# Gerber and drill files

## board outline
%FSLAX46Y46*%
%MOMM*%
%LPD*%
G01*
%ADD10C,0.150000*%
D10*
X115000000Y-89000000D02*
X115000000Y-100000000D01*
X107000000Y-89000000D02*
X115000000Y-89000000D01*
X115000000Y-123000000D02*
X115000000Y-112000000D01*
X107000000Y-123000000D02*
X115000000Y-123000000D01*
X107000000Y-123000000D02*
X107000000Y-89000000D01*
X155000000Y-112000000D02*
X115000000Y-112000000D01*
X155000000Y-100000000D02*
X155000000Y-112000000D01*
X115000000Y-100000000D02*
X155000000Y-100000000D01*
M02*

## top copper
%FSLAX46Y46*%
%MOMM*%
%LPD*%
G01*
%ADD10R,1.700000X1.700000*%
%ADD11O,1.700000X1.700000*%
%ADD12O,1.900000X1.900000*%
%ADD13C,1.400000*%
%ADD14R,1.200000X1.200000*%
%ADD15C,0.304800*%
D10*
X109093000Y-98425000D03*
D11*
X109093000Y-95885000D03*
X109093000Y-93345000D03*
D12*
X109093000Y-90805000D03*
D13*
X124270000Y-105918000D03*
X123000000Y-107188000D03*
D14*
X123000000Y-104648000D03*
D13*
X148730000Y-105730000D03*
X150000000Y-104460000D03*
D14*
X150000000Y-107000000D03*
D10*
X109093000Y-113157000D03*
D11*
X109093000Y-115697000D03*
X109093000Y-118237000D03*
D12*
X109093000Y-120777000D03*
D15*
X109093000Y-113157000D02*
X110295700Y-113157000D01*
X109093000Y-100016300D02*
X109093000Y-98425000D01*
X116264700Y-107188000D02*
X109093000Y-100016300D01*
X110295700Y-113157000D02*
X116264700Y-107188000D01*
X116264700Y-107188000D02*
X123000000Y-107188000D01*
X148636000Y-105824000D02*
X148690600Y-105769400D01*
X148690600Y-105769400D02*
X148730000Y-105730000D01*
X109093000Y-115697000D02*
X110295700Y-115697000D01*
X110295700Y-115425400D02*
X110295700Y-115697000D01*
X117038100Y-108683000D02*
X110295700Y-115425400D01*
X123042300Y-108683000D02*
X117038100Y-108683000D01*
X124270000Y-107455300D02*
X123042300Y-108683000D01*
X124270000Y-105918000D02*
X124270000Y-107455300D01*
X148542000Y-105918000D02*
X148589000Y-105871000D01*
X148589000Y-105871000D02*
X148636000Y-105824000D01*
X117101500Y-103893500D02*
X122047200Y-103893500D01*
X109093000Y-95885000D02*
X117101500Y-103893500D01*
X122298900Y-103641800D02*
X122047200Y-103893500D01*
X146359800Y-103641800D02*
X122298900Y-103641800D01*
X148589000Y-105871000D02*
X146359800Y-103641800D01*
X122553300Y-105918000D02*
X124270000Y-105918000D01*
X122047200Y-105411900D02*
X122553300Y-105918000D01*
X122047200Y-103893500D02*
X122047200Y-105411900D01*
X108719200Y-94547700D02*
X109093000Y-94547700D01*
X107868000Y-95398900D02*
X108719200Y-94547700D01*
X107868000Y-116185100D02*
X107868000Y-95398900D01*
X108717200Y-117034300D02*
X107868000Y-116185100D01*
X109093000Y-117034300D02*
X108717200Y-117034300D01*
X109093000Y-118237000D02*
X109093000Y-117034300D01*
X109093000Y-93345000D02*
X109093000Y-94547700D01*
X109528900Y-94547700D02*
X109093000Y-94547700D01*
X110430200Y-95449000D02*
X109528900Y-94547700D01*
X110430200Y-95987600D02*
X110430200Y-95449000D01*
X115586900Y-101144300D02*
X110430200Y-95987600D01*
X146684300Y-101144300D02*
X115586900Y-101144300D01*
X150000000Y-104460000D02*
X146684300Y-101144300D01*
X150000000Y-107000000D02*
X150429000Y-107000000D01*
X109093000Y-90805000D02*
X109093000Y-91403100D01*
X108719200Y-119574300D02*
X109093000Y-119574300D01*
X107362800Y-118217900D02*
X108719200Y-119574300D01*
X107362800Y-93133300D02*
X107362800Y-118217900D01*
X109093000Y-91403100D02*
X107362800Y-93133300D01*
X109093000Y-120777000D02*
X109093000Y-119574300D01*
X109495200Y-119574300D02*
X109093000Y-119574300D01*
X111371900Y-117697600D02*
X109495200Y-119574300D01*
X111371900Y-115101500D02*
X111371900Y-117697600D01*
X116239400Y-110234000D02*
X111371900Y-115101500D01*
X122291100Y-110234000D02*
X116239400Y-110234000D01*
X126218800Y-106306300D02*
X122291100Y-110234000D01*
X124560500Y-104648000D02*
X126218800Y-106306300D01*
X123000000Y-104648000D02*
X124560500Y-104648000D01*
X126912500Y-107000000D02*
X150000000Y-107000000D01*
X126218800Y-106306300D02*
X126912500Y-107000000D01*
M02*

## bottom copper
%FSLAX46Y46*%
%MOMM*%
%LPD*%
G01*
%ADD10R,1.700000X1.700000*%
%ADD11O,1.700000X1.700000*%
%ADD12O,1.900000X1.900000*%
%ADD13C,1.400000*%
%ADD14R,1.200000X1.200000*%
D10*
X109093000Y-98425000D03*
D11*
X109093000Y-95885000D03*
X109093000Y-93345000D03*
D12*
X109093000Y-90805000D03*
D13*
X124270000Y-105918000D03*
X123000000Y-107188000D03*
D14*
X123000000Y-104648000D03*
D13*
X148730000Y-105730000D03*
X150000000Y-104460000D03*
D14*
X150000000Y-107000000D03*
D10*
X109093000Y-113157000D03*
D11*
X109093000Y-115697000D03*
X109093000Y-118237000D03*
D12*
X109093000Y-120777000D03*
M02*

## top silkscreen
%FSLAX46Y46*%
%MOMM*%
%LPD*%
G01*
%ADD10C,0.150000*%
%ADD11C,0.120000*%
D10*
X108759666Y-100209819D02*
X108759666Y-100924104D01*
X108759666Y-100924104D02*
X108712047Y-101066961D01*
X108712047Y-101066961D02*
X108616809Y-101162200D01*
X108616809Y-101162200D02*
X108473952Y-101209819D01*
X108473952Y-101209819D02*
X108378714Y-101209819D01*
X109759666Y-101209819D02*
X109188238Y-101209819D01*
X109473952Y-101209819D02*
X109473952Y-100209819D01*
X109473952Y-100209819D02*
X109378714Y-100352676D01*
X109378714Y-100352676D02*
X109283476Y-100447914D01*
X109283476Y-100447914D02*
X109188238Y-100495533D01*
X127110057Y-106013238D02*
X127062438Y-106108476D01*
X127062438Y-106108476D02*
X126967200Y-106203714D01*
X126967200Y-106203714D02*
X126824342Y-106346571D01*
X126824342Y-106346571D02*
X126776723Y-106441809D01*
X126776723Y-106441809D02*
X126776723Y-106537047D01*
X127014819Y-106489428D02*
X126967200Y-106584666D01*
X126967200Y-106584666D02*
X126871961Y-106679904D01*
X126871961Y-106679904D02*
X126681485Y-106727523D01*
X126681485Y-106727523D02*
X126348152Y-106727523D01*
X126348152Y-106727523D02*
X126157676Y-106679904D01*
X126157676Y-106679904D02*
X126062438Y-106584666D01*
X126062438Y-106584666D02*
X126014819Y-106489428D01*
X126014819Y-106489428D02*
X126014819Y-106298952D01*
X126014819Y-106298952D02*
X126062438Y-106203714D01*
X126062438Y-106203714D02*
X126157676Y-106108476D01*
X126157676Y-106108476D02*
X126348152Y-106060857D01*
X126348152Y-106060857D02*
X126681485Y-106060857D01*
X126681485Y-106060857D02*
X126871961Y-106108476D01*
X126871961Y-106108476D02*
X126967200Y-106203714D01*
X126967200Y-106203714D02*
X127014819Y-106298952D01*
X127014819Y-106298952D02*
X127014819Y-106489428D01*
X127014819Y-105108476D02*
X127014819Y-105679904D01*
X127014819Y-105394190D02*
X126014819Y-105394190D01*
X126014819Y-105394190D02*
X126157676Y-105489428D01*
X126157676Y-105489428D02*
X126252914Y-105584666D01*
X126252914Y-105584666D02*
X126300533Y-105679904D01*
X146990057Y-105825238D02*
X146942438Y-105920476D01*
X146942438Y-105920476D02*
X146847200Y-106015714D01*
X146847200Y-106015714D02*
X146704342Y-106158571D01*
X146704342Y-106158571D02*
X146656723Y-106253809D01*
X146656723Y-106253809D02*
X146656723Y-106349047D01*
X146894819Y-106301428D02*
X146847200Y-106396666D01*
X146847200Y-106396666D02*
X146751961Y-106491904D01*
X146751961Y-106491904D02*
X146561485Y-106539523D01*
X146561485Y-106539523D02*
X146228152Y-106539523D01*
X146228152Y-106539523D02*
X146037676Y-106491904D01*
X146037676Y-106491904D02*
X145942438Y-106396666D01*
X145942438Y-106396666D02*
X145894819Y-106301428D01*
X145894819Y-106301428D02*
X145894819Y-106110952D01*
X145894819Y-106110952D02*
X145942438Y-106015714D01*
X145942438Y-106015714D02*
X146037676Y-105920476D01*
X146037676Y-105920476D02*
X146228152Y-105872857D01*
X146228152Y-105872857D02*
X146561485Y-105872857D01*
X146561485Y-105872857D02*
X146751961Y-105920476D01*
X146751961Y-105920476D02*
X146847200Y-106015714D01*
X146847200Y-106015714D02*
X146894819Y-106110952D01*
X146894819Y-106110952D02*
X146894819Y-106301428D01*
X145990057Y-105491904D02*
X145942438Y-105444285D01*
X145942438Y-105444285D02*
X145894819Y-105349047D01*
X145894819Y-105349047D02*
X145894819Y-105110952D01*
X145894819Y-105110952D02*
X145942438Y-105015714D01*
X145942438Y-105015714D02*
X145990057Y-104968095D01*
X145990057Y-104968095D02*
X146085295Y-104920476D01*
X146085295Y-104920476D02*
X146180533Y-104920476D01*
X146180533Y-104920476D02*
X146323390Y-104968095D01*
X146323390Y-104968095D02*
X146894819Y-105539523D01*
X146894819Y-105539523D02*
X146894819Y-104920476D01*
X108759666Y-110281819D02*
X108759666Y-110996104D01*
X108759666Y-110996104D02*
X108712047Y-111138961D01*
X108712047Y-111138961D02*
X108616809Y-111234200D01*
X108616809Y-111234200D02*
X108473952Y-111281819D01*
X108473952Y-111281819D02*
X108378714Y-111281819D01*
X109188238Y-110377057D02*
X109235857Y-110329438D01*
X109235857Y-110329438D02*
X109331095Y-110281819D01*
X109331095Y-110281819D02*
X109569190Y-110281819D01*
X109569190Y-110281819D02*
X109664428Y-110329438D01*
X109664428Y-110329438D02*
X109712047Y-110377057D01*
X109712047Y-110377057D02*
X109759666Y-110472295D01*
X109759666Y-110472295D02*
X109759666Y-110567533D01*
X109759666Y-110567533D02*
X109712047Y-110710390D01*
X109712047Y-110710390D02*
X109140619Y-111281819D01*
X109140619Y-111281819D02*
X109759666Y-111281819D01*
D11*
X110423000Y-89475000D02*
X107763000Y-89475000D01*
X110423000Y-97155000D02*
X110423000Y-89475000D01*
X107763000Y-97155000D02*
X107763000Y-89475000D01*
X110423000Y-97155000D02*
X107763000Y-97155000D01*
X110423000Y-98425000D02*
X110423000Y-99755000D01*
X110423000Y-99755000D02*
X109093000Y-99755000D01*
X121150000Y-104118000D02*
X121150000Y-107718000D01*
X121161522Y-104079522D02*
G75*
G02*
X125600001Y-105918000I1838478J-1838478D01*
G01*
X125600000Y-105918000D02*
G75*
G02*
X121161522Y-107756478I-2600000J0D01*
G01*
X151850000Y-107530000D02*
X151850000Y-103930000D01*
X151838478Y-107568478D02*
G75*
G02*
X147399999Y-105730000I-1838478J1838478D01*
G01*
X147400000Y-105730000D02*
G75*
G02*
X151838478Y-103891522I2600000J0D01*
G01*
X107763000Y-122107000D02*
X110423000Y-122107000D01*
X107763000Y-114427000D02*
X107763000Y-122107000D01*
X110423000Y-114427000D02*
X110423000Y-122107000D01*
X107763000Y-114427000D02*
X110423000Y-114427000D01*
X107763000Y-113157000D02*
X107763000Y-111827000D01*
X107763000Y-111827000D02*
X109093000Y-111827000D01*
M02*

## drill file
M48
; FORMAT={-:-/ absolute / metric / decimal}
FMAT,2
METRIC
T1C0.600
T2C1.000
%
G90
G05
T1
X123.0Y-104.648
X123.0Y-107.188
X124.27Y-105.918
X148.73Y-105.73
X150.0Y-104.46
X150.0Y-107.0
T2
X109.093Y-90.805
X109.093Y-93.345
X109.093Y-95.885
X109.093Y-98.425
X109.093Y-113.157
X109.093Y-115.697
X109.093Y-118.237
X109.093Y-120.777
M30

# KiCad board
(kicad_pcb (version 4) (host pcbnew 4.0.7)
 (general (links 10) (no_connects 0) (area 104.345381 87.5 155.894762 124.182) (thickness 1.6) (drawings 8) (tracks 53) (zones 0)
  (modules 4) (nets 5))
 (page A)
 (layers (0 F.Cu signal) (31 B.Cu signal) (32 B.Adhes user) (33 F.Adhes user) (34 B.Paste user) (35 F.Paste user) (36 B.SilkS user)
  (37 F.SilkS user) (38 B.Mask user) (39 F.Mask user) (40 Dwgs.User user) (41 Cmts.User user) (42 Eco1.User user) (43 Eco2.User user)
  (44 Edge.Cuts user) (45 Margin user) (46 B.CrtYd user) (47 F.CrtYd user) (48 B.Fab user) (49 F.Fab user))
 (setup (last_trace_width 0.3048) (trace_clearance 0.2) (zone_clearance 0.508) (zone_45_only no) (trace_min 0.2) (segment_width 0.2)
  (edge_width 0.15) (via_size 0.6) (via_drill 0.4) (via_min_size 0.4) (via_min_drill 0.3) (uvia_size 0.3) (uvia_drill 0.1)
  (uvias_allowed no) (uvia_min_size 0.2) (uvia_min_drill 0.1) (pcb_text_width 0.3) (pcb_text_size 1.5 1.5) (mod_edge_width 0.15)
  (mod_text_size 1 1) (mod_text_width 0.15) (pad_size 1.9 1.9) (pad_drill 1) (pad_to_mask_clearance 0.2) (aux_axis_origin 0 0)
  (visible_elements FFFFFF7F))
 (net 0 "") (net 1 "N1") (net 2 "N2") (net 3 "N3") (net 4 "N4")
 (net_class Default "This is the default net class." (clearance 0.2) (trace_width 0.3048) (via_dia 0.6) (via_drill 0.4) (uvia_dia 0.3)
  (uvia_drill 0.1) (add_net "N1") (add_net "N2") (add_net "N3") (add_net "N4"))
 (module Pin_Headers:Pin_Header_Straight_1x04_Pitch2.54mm (layer F.Cu) (at 109.093 98.425 180)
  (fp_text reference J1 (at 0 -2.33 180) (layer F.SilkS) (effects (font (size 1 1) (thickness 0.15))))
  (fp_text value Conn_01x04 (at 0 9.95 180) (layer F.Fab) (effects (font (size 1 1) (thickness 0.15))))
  (fp_line (start -1.33 8.95) (end 1.33 8.95) (layer F.SilkS) (width 0.12))
  (fp_line (start -1.33 1.27) (end -1.33 8.95) (layer F.SilkS) (width 0.12))
  (fp_line (start 1.33 1.27) (end 1.33 8.95) (layer F.SilkS) (width 0.12))
  (fp_line (start -1.33 1.27) (end 1.33 1.27) (layer F.SilkS) (width 0.12))
  (fp_line (start -1.33 0) (end -1.33 -1.33) (layer F.SilkS) (width 0.12))
  (fp_line (start -1.33 -1.33) (end 0 -1.33) (layer F.SilkS) (width 0.12))
  (pad 1 thru_hole rect (at 0 0 180) (size 1.7 1.7) (drill 1) (layers *.Cu *.Mask) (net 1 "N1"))
  (pad 2 thru_hole oval (at 0 2.54 180) (size 1.7 1.7) (drill 1) (layers *.Cu *.Mask) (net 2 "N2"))
  (pad 3 thru_hole oval (at 0 5.08 180) (size 1.7 1.7) (drill 1) (layers *.Cu *.Mask) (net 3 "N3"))
  (pad 4 thru_hole oval (at 0 7.62 180) (size 1.9 1.9) (drill 1) (layers *.Cu *.Mask) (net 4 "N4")))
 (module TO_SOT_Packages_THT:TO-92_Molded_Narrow (layer F.Cu) (at 123 104.648 270)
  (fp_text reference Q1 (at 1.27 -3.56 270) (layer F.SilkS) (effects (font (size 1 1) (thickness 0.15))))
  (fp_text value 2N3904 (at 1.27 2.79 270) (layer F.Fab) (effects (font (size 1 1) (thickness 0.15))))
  (fp_line (start -0.53 1.85) (end 3.07 1.85) (layer F.SilkS) (width 0.12))
  (fp_arc (start 1.27 0) (end 1.27 -2.6) (angle -135) (layer F.SilkS) (width 0.12))
  (fp_arc (start 1.27 0) (end 1.27 -2.6) (angle 135) (layer F.SilkS) (width 0.12))
  (pad 2 thru_hole circle (at 1.27 -1.27) (size 1.4 1.4) (drill 0.6) (layers *.Cu *.Mask) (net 2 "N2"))
  (pad 3 thru_hole circle (at 2.54 0) (size 1.4 1.4) (drill 0.6) (layers *.Cu *.Mask) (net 1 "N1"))
  (pad 1 thru_hole rect (at 0 0) (size 1.2 1.2) (drill 0.6) (layers *.Cu *.Mask) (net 4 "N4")))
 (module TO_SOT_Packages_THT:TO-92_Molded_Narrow (layer F.Cu) (at 150 107 90)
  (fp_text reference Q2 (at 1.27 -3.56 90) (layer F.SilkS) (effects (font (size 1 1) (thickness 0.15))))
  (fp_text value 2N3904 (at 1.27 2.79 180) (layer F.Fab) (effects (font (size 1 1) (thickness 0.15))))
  (fp_line (start -0.53 1.85) (end 3.07 1.85) (layer F.SilkS) (width 0.12))
  (fp_arc (start 1.27 0) (end 1.27 -2.6) (angle -135) (layer F.SilkS) (width 0.12))
  (fp_arc (start 1.27 0) (end 1.27 -2.6) (angle 135) (layer F.SilkS) (width 0.12))
  (pad 2 thru_hole circle (at 1.27 -1.27 180) (size 1.4 1.4) (drill 0.6) (layers *.Cu *.Mask) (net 2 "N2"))
  (pad 3 thru_hole circle (at 2.54 0 180) (size 1.4 1.4) (drill 0.6) (layers *.Cu *.Mask) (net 3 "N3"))
  (pad 1 thru_hole rect (at 0 0 180) (size 1.2 1.2) (drill 0.6) (layers *.Cu *.Mask) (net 4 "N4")))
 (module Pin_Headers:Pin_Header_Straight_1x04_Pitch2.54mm (layer F.Cu) (at 109.093 113.157)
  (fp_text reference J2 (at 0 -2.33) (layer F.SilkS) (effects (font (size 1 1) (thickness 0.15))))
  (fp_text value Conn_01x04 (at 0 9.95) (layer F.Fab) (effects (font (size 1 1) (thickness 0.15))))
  (fp_line (start -1.33 8.95) (end 1.33 8.95) (layer F.SilkS) (width 0.12))
  (fp_line (start -1.33 1.27) (end -1.33 8.95) (layer F.SilkS) (width 0.12))
  (fp_line (start 1.33 1.27) (end 1.33 8.95) (layer F.SilkS) (width 0.12))
  (fp_line (start -1.33 1.27) (end 1.33 1.27) (layer F.SilkS) (width 0.12))
  (fp_line (start -1.33 0) (end -1.33 -1.33) (layer F.SilkS) (width 0.12))
  (fp_line (start -1.33 -1.33) (end 0 -1.33) (layer F.SilkS) (width 0.12))
  (pad 1 thru_hole rect (at 0 0) (size 1.7 1.7) (drill 1) (layers *.Cu *.Mask) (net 1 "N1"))
  (pad 2 thru_hole oval (at 0 2.54) (size 1.7 1.7) (drill 1) (layers *.Cu *.Mask) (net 2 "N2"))
  (pad 3 thru_hole oval (at 0 5.08) (size 1.7 1.7) (drill 1) (layers *.Cu *.Mask) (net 3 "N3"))
  (pad 4 thru_hole oval (at 0 7.62) (size 1.9 1.9) (drill 1) (layers *.Cu *.Mask) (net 4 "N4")))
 (gr_line (start 115 89) (end 115 100) (angle 90) (layer Edge.Cuts) (width 0.15))
 (gr_line (start 107 89) (end 115 89) (angle 90) (layer Edge.Cuts) (width 0.15))
 (gr_line (start 115 123) (end 115 112) (angle 90) (layer Edge.Cuts) (width 0.15))
 (gr_line (start 107 123) (end 115 123) (angle 90) (layer Edge.Cuts) (width 0.15))
 (gr_line (start 107 123) (end 107 89) (angle 90) (layer Edge.Cuts) (width 0.15))
 (gr_line (start 155 112) (end 115 112) (angle 90) (layer Edge.Cuts) (width 0.15))
 (gr_line (start 155 100) (end 155 112) (angle 90) (layer Edge.Cuts) (width 0.15))
 (gr_line (start 115 100) (end 155 100) (angle 90) (layer Edge.Cuts) (width 0.15))
 (segment (start 109.093 113.157) (end 110.2957 113.157) (width 0.3048) (layer F.Cu) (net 1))
 (segment (start 109.093 100.0163) (end 109.093 98.425) (width 0.3048) (layer F.Cu) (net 1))
 (segment (start 116.2647 107.188) (end 109.093 100.0163) (width 0.3048) (layer F.Cu) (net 1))
 (segment (start 110.2957 113.157) (end 116.2647 107.188) (width 0.3048) (layer F.Cu) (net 1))
 (segment (start 116.2647 107.188) (end 123 107.188) (width 0.3048) (layer F.Cu) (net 1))
 (segment (start 148.636 105.824) (end 148.6906 105.7694) (width 0.3048) (layer F.Cu) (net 2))
 (segment (start 148.6906 105.7694) (end 148.73 105.73) (width 0.3048) (layer F.Cu) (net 2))
 (segment (start 109.093 115.697) (end 110.2957 115.697) (width 0.3048) (layer F.Cu) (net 2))
 (segment (start 110.2957 115.4254) (end 110.2957 115.697) (width 0.3048) (layer F.Cu) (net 2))
 (segment (start 117.0381 108.683) (end 110.2957 115.4254) (width 0.3048) (layer F.Cu) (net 2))
 (segment (start 123.0423 108.683) (end 117.0381 108.683) (width 0.3048) (layer F.Cu) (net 2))
 (segment (start 124.27 107.4553) (end 123.0423 108.683) (width 0.3048) (layer F.Cu) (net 2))
 (segment (start 124.27 105.918) (end 124.27 107.4553) (width 0.3048) (layer F.Cu) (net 2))
 (segment (start 148.542 105.918) (end 148.589 105.871) (width 0.3048) (layer F.Cu) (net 2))
 (segment (start 148.589 105.871) (end 148.636 105.824) (width 0.3048) (layer F.Cu) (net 2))
 (segment (start 117.1015 103.8935) (end 122.0472 103.8935) (width 0.3048) (layer F.Cu) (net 2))
 (segment (start 109.093 95.885) (end 117.1015 103.8935) (width 0.3048) (layer F.Cu) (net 2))
 (segment (start 122.2989 103.6418) (end 122.0472 103.8935) (width 0.3048) (layer F.Cu) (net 2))
 (segment (start 146.3598 103.6418) (end 122.2989 103.6418) (width 0.3048) (layer F.Cu) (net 2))
 (segment (start 148.589 105.871) (end 146.3598 103.6418) (width 0.3048) (layer F.Cu) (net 2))
 (segment (start 122.5533 105.918) (end 124.27 105.918) (width 0.3048) (layer F.Cu) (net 2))
 (segment (start 122.0472 105.4119) (end 122.5533 105.918) (width 0.3048) (layer F.Cu) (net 2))
 (segment (start 122.0472 103.8935) (end 122.0472 105.4119) (width 0.3048) (layer F.Cu) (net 2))
 (segment (start 108.7192 94.5477) (end 109.093 94.5477) (width 0.3048) (layer F.Cu) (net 3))
 (segment (start 107.868 95.3989) (end 108.7192 94.5477) (width 0.3048) (layer F.Cu) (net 3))
 (segment (start 107.868 116.1851) (end 107.868 95.3989) (width 0.3048) (layer F.Cu) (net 3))
 (segment (start 108.7172 117.0343) (end 107.868 116.1851) (width 0.3048) (layer F.Cu) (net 3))
 (segment (start 109.093 117.0343) (end 108.7172 117.0343) (width 0.3048) (layer F.Cu) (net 3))
 (segment (start 109.093 118.237) (end 109.093 117.0343) (width 0.3048) (layer F.Cu) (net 3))
 (segment (start 109.093 93.345) (end 109.093 94.5477) (width 0.3048) (layer F.Cu) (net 3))
 (segment (start 109.5289 94.5477) (end 109.093 94.5477) (width 0.3048) (layer F.Cu) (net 3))
 (segment (start 110.4302 95.449) (end 109.5289 94.5477) (width 0.3048) (layer F.Cu) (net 3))
 (segment (start 110.4302 95.9876) (end 110.4302 95.449) (width 0.3048) (layer F.Cu) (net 3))
 (segment (start 115.5869 101.1443) (end 110.4302 95.9876) (width 0.3048) (layer F.Cu) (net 3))
 (segment (start 146.6843 101.1443) (end 115.5869 101.1443) (width 0.3048) (layer F.Cu) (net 3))
 (segment (start 150 104.46) (end 146.6843 101.1443) (width 0.3048) (layer F.Cu) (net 3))
 (segment (start 150 107) (end 150.429 107) (width 0.3048) (layer F.Cu) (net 4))
 (segment (start 109.093 90.805) (end 109.093 91.4031) (width 0.3048) (layer F.Cu) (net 4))
 (segment (start 108.7192 119.5743) (end 109.093 119.5743) (width 0.3048) (layer F.Cu) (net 4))
 (segment (start 107.3628 118.2179) (end 108.7192 119.5743) (width 0.3048) (layer F.Cu) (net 4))
 (segment (start 107.3628 93.1333) (end 107.3628 118.2179) (width 0.3048) (layer F.Cu) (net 4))
 (segment (start 109.093 91.4031) (end 107.3628 93.1333) (width 0.3048) (layer F.Cu) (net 4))
 (segment (start 109.093 120.777) (end 109.093 119.5743) (width 0.3048) (layer F.Cu) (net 4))
 (segment (start 109.4952 119.5743) (end 109.093 119.5743) (width 0.3048) (layer F.Cu) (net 4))
 (segment (start 111.3719 117.6976) (end 109.4952 119.5743) (width 0.3048) (layer F.Cu) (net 4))
 (segment (start 111.3719 115.1015) (end 111.3719 117.6976) (width 0.3048) (layer F.Cu) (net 4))
 (segment (start 116.2394 110.234) (end 111.3719 115.1015) (width 0.3048) (layer F.Cu) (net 4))
 (segment (start 122.2911 110.234) (end 116.2394 110.234) (width 0.3048) (layer F.Cu) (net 4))
 (segment (start 126.2188 106.3063) (end 122.2911 110.234) (width 0.3048) (layer F.Cu) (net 4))
 (segment (start 124.5605 104.648) (end 126.2188 106.3063) (width 0.3048) (layer F.Cu) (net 4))
 (segment (start 123 104.648) (end 124.5605 104.648) (width 0.3048) (layer F.Cu) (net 4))
 (segment (start 126.9125 107) (end 150 107) (width 0.3048) (layer F.Cu) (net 4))
 (segment (start 126.2188 106.3063) (end 126.9125 107) (width 0.3048) (layer F.Cu) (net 4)))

